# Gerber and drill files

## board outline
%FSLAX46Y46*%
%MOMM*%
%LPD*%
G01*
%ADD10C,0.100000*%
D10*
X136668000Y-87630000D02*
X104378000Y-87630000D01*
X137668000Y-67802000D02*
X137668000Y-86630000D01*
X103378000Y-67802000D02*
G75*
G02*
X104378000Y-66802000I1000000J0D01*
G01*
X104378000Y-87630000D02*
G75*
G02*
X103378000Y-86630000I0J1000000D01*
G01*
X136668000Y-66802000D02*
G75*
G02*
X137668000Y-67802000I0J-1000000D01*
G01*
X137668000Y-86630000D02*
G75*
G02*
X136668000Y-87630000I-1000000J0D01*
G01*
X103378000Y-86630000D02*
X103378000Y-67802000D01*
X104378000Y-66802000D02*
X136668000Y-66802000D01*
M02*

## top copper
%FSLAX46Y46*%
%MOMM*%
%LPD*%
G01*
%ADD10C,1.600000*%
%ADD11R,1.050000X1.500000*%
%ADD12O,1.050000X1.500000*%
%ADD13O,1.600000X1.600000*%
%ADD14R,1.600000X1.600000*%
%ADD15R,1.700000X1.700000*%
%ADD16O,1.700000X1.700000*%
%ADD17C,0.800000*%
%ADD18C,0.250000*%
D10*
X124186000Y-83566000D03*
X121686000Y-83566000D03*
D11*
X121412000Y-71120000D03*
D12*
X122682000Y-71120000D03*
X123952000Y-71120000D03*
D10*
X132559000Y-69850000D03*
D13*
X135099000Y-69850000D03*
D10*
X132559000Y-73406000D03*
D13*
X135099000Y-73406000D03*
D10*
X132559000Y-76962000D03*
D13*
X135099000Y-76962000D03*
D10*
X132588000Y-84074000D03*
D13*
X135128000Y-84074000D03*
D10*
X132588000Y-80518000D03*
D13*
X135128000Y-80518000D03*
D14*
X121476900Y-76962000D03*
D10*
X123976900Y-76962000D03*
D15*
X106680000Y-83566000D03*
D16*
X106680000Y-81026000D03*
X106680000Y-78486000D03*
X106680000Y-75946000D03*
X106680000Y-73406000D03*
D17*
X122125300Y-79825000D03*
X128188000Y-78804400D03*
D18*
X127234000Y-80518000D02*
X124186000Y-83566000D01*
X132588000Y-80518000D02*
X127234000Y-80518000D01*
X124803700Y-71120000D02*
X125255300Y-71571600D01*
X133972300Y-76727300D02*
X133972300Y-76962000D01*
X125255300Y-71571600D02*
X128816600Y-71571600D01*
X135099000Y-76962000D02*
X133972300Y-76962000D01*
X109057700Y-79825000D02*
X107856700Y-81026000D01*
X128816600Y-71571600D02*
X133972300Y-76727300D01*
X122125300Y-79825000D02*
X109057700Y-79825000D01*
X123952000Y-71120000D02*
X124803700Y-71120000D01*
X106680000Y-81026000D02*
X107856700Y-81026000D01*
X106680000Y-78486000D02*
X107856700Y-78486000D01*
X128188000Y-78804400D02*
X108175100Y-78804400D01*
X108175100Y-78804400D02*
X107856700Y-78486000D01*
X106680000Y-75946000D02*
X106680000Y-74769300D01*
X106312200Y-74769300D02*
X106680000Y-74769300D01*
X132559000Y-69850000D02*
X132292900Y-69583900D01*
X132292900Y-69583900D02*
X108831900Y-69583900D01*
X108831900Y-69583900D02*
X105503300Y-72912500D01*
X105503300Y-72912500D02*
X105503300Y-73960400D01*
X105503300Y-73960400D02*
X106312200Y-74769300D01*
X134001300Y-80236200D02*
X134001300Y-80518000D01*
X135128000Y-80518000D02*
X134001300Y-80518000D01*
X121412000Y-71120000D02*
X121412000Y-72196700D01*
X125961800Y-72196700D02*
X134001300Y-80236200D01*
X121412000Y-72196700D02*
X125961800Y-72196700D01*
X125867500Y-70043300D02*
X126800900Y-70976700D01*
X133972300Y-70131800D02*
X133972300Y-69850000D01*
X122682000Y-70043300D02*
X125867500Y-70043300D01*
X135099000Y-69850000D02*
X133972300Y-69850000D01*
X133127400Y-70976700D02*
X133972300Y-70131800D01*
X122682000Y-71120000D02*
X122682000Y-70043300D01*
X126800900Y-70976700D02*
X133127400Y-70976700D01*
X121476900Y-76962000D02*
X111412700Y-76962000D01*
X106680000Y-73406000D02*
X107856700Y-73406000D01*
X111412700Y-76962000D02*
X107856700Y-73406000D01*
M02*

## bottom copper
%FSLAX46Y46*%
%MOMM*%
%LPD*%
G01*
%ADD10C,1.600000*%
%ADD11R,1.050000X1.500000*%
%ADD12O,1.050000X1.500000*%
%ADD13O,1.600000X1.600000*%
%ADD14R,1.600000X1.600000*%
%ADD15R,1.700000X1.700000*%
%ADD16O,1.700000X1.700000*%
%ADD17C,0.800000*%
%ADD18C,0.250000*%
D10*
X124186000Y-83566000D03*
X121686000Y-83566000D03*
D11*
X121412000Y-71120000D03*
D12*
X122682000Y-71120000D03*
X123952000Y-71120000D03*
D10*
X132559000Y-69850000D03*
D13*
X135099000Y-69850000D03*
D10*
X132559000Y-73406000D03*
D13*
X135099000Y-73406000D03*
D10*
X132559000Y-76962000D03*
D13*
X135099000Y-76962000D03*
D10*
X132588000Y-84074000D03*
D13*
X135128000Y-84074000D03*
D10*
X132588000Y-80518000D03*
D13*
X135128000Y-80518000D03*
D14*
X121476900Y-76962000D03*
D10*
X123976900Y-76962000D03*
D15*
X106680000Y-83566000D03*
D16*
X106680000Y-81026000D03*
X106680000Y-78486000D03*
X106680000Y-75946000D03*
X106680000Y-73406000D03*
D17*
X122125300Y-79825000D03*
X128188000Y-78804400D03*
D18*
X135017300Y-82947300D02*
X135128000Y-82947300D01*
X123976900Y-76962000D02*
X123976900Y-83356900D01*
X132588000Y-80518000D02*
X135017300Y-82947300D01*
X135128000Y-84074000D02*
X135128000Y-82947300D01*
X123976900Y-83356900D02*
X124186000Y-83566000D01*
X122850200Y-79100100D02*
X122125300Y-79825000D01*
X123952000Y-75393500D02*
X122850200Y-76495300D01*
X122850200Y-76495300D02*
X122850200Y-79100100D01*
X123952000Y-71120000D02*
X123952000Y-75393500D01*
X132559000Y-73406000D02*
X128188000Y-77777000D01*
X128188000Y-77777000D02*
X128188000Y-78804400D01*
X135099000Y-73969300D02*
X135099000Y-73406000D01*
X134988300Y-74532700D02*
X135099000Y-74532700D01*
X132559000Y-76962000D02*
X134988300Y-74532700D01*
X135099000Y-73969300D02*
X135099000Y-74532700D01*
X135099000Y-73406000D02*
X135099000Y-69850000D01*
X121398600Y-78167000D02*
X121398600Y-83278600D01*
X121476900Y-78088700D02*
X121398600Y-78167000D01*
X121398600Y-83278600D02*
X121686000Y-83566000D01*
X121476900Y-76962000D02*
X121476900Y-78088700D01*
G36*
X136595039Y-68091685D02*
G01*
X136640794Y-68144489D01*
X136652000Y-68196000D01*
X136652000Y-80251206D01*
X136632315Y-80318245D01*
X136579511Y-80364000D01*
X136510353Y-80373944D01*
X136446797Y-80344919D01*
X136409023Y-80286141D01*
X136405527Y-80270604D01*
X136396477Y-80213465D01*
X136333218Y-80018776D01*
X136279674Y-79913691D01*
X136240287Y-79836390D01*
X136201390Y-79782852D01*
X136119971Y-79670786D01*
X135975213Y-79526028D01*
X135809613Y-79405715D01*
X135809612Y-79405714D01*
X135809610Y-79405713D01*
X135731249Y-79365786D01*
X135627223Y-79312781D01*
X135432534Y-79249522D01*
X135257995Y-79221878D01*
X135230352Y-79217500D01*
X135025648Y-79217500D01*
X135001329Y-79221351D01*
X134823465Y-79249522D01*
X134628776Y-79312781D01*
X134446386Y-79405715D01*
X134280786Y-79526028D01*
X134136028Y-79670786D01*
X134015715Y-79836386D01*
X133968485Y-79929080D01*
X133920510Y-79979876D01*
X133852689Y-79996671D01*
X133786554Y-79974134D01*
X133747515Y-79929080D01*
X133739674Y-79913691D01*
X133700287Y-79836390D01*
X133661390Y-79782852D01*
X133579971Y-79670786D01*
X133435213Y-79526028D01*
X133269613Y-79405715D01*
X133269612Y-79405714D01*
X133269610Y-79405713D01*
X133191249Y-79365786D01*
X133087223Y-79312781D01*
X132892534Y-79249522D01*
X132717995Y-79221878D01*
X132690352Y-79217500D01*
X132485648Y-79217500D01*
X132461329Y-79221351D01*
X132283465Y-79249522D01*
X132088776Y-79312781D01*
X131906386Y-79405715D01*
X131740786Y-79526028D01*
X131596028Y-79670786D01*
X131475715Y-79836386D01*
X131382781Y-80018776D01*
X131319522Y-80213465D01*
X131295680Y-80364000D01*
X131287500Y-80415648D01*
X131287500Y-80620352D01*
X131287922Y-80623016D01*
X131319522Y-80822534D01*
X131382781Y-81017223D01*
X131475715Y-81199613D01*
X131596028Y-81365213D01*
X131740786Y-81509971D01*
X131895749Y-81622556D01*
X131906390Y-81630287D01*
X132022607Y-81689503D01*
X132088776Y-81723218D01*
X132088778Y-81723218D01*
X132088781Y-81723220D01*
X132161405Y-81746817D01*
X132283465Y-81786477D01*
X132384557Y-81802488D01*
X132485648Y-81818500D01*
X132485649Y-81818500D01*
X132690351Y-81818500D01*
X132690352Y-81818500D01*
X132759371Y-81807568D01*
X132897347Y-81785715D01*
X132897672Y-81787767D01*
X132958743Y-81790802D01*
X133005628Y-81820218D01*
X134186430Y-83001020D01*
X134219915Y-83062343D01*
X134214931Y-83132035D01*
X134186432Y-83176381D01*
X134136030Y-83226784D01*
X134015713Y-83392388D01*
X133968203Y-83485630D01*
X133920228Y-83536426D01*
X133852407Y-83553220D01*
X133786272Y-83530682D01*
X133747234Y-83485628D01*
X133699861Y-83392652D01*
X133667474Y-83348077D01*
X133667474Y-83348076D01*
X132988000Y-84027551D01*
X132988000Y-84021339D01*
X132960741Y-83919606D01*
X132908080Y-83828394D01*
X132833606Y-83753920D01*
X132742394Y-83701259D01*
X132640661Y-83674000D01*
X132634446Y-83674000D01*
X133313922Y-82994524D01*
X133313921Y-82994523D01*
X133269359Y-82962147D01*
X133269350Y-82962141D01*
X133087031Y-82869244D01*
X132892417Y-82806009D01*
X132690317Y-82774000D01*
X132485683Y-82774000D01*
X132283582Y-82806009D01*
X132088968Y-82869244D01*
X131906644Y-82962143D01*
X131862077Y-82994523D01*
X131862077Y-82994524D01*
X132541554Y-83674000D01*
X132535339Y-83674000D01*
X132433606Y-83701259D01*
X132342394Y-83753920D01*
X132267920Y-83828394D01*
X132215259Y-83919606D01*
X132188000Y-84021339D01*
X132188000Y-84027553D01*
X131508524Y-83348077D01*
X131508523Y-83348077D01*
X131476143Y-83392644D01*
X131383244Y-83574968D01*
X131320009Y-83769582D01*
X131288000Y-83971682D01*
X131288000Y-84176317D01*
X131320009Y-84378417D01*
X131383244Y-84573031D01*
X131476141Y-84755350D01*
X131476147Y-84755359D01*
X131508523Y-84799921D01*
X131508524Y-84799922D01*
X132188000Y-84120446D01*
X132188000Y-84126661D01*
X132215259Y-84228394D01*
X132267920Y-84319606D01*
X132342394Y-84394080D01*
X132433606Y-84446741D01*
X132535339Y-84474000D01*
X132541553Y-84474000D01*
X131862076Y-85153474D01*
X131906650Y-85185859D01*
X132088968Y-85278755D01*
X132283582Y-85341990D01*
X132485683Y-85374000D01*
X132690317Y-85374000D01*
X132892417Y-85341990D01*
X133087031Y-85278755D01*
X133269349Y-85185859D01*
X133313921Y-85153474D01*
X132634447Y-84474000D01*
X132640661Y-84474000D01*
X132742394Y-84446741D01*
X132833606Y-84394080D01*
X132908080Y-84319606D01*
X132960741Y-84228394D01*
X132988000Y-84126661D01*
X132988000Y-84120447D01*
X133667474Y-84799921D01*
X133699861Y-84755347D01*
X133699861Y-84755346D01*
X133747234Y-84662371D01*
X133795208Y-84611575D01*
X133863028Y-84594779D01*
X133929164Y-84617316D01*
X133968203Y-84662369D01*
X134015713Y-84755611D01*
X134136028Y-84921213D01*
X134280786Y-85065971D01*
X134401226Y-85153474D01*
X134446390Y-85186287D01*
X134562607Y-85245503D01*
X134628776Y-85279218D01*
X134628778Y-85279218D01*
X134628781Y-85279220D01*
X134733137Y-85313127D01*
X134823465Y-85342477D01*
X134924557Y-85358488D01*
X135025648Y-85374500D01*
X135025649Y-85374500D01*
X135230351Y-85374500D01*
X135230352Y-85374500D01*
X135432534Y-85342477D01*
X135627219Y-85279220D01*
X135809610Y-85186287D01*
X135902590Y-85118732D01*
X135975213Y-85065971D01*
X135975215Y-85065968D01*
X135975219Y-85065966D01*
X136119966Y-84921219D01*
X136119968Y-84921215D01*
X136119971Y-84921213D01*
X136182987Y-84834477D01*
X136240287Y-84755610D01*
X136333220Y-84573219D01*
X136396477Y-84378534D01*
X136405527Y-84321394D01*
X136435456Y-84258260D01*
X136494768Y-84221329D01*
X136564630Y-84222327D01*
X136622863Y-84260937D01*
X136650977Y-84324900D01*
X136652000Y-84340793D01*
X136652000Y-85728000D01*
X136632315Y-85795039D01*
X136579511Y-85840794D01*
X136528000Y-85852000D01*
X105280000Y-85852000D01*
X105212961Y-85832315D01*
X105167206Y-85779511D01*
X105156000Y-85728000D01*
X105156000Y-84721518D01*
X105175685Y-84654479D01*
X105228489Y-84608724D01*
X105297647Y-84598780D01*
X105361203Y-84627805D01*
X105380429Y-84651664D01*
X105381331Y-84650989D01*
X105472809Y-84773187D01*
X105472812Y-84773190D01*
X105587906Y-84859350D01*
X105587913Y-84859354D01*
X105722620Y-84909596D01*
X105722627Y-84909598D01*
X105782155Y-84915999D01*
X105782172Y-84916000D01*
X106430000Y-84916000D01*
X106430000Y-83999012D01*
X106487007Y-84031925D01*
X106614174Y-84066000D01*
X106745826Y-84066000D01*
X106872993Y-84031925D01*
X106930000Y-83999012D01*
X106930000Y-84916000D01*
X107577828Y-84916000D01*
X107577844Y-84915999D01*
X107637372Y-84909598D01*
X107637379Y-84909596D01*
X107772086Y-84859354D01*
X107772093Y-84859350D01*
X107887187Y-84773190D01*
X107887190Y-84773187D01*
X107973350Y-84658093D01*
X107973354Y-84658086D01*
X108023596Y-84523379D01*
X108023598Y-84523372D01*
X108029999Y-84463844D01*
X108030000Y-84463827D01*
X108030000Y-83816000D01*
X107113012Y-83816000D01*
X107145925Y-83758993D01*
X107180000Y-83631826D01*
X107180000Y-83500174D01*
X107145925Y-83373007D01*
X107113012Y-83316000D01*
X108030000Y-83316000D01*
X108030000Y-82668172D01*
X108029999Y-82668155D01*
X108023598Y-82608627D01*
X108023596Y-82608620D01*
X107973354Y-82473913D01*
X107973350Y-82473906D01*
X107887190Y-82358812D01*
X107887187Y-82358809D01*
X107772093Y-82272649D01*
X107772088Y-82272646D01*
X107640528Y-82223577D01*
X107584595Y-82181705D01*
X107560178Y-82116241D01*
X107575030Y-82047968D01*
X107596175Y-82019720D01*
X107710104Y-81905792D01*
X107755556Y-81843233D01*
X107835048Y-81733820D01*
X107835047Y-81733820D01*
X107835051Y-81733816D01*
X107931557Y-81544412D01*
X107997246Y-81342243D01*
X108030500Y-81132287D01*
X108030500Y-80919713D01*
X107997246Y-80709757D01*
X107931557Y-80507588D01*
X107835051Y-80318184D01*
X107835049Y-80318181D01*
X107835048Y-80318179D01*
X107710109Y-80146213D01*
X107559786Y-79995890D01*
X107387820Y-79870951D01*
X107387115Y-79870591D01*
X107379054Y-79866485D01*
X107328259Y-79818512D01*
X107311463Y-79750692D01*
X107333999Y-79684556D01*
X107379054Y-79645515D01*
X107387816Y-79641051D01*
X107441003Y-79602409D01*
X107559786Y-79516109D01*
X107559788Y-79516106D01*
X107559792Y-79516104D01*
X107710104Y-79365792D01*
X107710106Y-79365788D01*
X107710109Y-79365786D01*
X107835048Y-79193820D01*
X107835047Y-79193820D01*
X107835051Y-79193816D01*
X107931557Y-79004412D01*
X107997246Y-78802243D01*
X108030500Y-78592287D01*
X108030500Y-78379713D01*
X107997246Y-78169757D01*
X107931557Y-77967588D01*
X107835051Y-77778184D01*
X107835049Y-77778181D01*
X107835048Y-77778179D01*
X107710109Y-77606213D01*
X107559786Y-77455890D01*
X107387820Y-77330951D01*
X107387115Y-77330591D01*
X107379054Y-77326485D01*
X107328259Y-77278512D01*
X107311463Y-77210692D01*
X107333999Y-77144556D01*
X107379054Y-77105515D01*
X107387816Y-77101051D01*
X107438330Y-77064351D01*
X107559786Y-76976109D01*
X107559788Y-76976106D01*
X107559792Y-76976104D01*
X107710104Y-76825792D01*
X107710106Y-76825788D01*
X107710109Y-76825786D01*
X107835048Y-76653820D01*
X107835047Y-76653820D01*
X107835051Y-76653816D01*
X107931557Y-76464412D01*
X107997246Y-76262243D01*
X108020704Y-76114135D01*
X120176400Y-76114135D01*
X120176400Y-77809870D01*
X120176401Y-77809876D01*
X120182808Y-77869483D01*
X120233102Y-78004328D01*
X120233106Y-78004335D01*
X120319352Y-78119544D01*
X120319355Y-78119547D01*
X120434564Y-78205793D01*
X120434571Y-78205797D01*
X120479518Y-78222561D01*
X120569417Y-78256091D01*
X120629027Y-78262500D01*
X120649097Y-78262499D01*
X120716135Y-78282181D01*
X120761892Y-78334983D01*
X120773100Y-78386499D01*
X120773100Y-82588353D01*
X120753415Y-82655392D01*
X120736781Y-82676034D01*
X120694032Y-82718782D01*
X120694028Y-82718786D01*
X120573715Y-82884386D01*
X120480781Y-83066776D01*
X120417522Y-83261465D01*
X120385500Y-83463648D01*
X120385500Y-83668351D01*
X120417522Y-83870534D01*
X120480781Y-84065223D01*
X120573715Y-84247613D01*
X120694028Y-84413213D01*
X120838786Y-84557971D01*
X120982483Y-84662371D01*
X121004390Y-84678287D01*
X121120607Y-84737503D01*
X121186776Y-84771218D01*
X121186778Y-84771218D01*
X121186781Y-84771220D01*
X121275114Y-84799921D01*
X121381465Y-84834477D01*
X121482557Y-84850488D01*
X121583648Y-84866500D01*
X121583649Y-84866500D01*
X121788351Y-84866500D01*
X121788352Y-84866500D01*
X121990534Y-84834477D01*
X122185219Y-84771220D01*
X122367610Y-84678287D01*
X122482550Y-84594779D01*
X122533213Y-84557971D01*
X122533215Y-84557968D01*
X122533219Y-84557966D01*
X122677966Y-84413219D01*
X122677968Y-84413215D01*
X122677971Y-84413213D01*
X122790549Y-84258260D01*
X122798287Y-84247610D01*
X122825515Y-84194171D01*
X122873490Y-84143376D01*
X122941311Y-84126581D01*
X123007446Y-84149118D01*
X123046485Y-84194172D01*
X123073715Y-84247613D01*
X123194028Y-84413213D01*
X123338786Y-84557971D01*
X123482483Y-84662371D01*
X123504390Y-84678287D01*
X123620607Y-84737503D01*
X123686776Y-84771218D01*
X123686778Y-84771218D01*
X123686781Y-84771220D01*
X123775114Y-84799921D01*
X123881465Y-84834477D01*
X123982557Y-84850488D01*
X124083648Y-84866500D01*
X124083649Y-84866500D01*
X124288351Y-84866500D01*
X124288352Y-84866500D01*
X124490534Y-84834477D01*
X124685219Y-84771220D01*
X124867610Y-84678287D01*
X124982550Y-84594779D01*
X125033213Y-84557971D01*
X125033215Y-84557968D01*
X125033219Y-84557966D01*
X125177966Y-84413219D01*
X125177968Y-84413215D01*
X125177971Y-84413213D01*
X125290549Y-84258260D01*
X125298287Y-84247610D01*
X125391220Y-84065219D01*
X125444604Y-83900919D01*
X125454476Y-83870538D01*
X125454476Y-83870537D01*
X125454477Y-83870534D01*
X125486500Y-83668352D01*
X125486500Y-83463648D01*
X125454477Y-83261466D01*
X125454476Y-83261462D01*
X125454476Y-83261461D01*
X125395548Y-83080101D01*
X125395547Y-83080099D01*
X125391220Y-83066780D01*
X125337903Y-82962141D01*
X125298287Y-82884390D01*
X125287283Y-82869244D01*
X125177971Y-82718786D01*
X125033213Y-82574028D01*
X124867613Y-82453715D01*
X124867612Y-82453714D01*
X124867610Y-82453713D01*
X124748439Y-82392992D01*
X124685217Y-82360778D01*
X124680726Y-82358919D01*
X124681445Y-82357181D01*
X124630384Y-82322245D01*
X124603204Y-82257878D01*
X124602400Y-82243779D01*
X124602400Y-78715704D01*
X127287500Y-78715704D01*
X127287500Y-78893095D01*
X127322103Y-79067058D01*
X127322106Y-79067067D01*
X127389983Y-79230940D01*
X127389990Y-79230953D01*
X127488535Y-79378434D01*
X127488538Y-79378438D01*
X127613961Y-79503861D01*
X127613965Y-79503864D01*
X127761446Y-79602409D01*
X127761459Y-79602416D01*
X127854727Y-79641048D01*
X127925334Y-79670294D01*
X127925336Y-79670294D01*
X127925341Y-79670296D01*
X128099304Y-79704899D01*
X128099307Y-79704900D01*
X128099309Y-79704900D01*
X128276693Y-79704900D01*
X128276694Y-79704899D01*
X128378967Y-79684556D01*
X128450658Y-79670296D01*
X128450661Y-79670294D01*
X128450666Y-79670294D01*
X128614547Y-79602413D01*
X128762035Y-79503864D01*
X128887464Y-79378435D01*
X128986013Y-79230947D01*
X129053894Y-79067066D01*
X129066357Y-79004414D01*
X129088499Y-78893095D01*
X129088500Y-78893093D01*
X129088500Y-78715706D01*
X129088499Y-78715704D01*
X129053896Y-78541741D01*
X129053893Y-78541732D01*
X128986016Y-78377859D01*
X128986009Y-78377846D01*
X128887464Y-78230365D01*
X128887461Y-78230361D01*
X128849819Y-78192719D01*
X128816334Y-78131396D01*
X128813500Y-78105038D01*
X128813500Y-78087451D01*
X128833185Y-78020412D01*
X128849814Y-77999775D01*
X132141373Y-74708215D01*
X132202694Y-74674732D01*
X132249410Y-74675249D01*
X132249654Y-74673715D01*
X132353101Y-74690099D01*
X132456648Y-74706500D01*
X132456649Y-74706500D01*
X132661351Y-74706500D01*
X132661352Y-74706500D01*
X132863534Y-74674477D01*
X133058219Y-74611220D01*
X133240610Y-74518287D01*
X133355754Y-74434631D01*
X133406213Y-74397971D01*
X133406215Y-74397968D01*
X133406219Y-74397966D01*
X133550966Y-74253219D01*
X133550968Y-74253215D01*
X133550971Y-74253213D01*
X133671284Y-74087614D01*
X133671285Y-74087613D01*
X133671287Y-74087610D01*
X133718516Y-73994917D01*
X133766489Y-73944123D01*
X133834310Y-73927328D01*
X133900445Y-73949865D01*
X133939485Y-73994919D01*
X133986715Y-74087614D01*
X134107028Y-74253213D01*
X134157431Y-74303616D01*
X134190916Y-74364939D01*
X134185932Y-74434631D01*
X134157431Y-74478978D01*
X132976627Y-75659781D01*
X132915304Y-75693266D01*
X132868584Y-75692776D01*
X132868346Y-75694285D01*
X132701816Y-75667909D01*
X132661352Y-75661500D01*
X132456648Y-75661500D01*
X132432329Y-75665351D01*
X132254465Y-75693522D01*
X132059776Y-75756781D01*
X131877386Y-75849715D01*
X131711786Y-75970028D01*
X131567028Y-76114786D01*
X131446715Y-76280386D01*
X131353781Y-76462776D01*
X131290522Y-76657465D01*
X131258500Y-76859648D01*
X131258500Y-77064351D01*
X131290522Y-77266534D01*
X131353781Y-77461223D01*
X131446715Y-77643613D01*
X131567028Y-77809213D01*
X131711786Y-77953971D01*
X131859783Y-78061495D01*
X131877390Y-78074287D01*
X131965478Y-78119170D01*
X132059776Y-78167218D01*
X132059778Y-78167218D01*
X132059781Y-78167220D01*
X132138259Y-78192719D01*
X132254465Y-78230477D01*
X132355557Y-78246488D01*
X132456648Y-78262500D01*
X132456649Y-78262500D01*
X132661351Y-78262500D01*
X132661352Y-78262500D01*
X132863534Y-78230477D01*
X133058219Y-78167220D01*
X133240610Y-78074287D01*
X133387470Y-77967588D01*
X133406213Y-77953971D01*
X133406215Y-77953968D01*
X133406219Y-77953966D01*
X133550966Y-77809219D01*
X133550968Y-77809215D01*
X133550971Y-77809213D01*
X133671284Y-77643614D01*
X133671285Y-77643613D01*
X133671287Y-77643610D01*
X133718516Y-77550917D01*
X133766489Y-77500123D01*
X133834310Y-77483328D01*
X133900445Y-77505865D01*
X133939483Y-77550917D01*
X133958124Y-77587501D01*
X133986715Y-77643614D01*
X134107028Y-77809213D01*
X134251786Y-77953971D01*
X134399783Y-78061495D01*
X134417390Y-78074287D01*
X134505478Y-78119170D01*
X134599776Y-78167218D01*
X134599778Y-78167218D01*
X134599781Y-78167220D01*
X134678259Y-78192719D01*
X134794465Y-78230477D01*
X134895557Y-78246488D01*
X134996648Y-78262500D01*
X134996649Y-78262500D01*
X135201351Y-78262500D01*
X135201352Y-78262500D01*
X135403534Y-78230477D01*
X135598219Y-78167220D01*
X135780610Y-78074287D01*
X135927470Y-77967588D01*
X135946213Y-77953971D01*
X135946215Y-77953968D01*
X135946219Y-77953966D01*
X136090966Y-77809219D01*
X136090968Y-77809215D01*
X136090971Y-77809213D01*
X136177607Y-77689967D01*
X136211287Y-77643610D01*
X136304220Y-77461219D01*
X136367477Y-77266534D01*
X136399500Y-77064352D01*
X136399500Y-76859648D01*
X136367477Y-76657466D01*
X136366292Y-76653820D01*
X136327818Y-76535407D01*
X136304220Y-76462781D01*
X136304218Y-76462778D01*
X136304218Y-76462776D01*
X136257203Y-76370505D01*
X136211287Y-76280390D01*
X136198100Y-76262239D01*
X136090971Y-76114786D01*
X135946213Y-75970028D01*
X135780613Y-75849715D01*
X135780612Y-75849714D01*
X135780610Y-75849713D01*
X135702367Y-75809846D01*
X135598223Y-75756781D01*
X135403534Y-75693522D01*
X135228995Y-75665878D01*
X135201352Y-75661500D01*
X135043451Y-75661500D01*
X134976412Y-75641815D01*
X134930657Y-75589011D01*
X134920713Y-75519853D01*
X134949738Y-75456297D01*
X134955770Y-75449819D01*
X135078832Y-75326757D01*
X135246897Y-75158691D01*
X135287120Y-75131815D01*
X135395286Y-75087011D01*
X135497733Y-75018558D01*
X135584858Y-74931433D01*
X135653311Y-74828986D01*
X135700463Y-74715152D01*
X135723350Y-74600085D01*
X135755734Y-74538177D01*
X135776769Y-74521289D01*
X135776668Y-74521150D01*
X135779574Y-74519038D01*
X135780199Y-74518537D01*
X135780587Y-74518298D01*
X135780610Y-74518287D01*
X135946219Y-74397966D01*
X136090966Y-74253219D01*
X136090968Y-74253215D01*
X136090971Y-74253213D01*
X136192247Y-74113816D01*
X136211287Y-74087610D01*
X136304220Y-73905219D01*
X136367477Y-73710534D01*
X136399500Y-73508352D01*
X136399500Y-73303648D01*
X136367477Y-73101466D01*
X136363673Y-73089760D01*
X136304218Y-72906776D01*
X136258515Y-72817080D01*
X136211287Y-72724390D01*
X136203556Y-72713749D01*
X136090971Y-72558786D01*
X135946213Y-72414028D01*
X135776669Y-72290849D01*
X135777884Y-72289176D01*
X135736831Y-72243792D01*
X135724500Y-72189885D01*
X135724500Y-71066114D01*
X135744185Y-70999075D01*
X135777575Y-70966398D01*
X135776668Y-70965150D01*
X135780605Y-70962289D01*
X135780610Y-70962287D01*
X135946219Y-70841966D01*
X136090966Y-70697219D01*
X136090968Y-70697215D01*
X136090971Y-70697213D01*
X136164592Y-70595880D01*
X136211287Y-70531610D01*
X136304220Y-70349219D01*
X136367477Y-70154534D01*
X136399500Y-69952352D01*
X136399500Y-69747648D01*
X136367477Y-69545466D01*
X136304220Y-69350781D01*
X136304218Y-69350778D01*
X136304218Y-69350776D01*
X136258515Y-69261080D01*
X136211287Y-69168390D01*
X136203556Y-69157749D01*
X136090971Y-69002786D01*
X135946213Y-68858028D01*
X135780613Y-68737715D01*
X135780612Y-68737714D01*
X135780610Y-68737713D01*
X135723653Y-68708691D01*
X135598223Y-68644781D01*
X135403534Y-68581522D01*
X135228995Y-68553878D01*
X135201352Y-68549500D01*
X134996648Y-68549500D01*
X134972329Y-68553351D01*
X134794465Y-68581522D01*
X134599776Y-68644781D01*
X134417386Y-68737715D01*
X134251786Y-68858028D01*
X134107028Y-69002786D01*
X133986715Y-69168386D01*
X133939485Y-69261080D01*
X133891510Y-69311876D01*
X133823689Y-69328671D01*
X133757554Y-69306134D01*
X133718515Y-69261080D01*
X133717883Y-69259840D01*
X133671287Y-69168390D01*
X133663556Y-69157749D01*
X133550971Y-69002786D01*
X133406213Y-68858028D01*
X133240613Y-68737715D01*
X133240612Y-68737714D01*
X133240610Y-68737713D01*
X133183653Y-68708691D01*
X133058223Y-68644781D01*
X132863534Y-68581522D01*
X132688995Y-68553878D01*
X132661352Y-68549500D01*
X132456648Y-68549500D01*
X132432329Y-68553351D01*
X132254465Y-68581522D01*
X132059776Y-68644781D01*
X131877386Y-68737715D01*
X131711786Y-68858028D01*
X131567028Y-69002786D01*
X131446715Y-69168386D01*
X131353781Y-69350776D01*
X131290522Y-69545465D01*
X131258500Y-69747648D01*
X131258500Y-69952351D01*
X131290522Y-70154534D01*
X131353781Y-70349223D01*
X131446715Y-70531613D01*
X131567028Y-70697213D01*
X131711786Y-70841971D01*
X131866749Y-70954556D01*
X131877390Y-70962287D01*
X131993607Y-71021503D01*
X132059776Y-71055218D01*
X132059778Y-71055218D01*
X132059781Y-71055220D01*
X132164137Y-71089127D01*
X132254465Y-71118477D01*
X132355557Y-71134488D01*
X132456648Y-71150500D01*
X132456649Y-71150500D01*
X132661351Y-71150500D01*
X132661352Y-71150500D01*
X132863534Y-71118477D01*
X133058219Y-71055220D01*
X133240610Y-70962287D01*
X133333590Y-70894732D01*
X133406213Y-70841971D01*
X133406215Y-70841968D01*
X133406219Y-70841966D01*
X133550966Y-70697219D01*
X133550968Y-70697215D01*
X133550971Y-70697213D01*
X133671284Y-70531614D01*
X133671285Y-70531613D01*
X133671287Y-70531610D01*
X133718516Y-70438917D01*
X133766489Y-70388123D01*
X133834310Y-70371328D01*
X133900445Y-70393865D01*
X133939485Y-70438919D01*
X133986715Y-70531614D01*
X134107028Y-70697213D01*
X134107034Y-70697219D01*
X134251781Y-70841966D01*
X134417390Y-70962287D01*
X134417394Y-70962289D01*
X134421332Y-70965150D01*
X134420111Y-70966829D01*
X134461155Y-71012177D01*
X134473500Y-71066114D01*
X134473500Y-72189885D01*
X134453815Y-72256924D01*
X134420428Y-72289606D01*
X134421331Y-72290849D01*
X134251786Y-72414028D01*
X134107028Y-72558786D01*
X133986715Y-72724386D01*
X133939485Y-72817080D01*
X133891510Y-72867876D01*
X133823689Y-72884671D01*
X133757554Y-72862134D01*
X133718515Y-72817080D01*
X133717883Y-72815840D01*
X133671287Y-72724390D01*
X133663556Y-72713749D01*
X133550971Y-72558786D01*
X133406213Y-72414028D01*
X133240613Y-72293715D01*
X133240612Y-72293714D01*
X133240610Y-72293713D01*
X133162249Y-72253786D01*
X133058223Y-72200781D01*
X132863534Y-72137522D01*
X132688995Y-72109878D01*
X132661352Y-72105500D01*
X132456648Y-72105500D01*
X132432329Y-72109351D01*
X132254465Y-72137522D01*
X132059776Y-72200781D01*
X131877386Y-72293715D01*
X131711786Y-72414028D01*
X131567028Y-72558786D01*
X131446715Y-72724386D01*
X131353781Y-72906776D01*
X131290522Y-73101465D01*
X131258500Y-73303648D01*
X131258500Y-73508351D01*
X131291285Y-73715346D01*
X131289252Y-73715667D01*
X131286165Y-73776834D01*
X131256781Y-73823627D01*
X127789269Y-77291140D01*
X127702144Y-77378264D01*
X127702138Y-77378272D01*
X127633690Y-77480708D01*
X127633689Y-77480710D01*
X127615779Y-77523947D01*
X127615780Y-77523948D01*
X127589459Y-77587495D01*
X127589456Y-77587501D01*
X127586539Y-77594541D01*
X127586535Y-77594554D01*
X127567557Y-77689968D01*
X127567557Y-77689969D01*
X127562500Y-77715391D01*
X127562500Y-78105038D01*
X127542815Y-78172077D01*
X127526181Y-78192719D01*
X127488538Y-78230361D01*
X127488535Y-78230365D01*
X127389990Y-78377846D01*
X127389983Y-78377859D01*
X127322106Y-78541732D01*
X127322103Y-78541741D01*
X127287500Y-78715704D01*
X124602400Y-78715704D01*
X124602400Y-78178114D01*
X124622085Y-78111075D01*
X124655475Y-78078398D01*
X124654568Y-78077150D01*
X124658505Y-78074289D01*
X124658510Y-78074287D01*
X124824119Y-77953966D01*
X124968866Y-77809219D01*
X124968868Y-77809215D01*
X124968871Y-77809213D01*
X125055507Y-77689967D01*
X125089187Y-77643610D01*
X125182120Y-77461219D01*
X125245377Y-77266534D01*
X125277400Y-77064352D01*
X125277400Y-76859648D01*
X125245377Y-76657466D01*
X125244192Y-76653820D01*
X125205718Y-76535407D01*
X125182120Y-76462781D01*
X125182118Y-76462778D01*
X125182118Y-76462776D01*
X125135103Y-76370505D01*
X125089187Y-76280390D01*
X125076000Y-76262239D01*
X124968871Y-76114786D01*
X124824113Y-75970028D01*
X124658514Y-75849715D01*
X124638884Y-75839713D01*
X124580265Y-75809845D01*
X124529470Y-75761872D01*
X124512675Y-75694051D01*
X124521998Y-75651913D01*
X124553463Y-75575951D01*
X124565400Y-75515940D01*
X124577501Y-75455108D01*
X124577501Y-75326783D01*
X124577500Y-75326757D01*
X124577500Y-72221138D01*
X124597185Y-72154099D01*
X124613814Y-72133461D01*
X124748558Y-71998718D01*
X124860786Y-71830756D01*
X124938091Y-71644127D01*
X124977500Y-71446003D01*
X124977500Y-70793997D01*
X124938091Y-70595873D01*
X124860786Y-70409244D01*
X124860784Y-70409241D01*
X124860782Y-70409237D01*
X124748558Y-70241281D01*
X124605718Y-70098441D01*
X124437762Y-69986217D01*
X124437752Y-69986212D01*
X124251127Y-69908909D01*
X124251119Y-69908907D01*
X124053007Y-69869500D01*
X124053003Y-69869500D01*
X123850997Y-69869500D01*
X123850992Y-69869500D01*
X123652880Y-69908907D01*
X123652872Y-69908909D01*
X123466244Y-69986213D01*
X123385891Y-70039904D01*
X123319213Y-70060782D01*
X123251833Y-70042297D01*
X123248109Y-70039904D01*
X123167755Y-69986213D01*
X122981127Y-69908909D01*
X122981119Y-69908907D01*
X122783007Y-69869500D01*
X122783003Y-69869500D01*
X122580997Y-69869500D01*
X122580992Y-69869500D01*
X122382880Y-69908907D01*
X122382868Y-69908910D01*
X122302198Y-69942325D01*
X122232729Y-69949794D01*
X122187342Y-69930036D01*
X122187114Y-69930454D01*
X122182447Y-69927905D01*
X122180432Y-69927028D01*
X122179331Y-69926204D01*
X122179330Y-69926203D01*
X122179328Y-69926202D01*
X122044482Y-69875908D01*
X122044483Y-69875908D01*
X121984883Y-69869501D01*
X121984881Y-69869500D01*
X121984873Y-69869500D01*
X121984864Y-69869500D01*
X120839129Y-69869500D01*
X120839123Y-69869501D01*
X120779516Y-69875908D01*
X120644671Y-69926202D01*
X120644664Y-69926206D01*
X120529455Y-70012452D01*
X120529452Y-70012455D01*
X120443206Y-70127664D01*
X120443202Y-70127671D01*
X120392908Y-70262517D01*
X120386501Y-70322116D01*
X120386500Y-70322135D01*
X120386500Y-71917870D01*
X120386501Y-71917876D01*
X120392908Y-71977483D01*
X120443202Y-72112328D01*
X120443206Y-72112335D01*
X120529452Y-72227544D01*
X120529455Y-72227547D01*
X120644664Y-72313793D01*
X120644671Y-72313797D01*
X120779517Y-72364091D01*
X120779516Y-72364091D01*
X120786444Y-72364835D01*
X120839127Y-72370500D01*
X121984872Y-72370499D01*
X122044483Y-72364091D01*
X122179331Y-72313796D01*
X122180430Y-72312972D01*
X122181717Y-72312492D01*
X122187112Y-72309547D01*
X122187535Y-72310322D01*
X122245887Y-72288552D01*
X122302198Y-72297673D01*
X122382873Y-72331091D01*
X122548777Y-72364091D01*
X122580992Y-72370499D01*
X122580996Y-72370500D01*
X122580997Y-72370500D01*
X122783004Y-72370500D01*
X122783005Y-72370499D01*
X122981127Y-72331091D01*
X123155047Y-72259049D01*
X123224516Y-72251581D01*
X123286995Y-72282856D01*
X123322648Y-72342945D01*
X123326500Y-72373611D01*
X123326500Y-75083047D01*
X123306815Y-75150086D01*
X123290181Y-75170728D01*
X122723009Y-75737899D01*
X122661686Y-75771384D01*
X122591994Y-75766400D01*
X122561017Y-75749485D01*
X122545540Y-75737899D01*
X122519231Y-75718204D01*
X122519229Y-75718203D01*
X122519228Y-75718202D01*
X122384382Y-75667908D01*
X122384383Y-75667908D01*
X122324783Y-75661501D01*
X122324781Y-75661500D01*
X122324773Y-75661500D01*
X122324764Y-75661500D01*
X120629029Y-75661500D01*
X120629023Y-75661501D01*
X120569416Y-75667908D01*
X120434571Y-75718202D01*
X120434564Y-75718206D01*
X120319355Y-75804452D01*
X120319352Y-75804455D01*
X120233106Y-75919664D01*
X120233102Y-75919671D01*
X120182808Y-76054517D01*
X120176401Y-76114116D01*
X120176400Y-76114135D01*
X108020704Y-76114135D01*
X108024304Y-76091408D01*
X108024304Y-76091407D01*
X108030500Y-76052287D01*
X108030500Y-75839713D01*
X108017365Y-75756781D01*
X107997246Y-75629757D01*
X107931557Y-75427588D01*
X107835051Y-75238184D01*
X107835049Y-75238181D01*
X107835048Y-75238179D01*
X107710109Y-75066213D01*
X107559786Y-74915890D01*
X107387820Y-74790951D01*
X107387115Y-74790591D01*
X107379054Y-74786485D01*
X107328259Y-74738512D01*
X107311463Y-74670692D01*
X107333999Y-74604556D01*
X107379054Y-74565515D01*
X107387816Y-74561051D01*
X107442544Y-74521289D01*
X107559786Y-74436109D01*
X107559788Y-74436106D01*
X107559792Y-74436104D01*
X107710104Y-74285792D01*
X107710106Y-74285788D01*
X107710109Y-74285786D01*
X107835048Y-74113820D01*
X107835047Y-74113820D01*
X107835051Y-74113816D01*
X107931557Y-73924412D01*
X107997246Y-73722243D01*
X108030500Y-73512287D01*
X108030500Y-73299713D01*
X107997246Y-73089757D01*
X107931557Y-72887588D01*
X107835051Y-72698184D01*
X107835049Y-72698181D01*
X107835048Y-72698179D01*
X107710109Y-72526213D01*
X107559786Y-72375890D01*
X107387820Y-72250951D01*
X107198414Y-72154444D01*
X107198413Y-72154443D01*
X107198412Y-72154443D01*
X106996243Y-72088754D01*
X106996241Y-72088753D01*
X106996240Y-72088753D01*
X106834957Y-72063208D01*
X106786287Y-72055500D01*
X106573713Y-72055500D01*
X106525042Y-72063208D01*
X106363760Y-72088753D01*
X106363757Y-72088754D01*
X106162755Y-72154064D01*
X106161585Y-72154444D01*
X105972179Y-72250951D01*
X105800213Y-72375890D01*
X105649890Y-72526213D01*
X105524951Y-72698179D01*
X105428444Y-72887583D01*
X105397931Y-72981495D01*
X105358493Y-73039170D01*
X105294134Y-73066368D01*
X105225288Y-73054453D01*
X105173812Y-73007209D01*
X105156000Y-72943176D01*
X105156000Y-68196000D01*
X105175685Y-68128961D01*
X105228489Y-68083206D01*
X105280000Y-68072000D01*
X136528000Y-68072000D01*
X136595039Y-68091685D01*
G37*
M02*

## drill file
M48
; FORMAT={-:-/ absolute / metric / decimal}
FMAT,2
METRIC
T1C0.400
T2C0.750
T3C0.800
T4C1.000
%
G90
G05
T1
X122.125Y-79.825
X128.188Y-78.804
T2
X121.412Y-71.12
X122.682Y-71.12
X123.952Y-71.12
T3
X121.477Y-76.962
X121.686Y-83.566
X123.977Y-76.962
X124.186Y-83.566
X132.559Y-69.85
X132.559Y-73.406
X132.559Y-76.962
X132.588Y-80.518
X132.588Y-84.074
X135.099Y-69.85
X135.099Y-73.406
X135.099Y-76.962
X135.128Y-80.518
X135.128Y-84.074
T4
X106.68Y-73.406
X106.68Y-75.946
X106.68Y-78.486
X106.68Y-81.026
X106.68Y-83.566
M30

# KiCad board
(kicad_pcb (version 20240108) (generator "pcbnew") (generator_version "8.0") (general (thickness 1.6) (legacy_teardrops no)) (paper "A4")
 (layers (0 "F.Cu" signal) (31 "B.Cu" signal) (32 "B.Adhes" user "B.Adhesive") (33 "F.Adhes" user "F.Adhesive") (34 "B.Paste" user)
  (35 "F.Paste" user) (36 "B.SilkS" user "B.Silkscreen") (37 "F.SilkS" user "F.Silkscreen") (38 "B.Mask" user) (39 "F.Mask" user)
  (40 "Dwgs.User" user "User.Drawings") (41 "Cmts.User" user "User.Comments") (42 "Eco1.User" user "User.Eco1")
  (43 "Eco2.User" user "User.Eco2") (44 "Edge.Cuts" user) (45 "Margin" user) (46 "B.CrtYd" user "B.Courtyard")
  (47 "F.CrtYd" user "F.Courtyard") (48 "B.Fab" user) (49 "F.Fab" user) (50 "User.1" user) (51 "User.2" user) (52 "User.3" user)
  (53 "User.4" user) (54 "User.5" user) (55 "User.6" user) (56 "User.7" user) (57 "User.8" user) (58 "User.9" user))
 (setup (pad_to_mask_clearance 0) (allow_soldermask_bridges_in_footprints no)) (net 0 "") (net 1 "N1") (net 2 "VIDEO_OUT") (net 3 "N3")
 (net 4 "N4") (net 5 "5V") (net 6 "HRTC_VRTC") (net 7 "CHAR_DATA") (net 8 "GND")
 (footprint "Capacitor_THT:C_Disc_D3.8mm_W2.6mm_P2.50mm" (layer "F.Cu") (at 124.186 83.566 180)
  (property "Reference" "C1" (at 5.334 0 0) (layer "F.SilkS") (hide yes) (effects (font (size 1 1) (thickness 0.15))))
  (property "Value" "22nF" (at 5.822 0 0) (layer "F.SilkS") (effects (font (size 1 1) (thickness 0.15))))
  (pad "1" thru_hole circle (at 0 0 180) (size 1.6 1.6) (drill 0.8) (layers "*.Cu" "*.Mask") (remove_unused_layers no) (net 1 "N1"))
  (pad "2" thru_hole circle (at 2.5 0 180) (size 1.6 1.6) (drill 0.8) (layers "*.Cu" "*.Mask") (remove_unused_layers no) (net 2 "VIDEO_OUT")))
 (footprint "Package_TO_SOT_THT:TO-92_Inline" (layer "F.Cu") (at 121.412 71.12)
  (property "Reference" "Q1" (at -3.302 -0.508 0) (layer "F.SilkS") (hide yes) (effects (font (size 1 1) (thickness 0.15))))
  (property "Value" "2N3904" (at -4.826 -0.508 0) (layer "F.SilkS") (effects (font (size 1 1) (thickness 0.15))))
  (pad "1" thru_hole rect (at 0 0) (size 1.05 1.5) (drill 0.75) (layers "*.Cu" "*.Mask") (remove_unused_layers no) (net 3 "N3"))
  (pad "2" thru_hole oval (at 1.27 0) (size 1.05 1.5) (drill 0.75) (layers "*.Cu" "*.Mask") (remove_unused_layers no) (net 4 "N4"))
  (pad "3" thru_hole oval (at 2.54 0) (size 1.05 1.5) (drill 0.75) (layers "*.Cu" "*.Mask") (remove_unused_layers no) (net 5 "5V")))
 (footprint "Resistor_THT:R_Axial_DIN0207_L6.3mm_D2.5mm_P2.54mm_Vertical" (layer "F.Cu") (at 132.559 69.85)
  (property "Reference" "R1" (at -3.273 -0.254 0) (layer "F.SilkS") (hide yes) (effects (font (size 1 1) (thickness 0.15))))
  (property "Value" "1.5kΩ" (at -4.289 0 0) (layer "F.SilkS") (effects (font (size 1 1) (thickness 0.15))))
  (pad "1" thru_hole circle (at 0 0) (size 1.6 1.6) (drill 0.8) (layers "*.Cu" "*.Mask") (remove_unused_layers no) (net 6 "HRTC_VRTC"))
  (pad "2" thru_hole oval (at 2.54 0) (size 1.6 1.6) (drill 0.8) (layers "*.Cu" "*.Mask") (remove_unused_layers no) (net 4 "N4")))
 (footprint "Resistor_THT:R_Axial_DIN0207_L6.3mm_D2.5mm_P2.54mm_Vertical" (layer "F.Cu") (at 132.559 73.406)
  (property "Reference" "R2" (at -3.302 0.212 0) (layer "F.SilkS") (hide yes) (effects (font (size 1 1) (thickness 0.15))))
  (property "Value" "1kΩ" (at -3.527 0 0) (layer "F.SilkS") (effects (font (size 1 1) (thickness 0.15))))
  (pad "1" thru_hole circle (at 0 0) (size 1.6 1.6) (drill 0.8) (layers "*.Cu" "*.Mask") (remove_unused_layers no) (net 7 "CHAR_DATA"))
  (pad "2" thru_hole oval (at 2.54 0) (size 1.6 1.6) (drill 0.8) (layers "*.Cu" "*.Mask") (remove_unused_layers no) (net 4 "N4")))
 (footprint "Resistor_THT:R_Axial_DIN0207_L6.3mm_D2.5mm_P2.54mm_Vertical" (layer "F.Cu") (at 132.559 76.962)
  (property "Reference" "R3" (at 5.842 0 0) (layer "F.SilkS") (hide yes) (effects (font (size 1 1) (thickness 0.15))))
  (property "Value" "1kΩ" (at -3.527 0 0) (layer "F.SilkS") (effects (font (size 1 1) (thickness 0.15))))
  (pad "1" thru_hole circle (at 0 0) (size 1.6 1.6) (drill 0.8) (layers "*.Cu" "*.Mask") (remove_unused_layers no) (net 4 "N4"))
  (pad "2" thru_hole oval (at 2.54 0) (size 1.6 1.6) (drill 0.8) (layers "*.Cu" "*.Mask") (remove_unused_layers no) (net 5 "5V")))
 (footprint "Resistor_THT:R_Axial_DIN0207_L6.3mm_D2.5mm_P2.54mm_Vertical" (layer "F.Cu") (at 132.588 84.074)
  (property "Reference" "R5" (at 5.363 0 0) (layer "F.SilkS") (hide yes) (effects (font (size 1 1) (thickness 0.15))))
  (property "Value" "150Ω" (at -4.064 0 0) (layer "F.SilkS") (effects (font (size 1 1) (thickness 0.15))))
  (pad "1" thru_hole circle (at 0 0) (size 1.6 1.6) (drill 0.8) (layers "*.Cu" "*.Mask") (remove_unused_layers no) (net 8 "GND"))
  (pad "2" thru_hole oval (at 2.54 0) (size 1.6 1.6) (drill 0.8) (layers "*.Cu" "*.Mask") (remove_unused_layers no) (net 1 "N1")))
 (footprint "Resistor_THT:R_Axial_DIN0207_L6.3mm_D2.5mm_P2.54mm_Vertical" (layer "F.Cu") (at 132.588 80.518)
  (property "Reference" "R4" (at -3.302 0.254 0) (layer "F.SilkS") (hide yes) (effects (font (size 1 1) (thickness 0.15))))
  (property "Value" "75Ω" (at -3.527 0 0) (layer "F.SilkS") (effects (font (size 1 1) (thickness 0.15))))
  (pad "1" thru_hole circle (at 0 0) (size 1.6 1.6) (drill 0.8) (layers "*.Cu" "*.Mask") (remove_unused_layers no) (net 1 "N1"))
  (pad "2" thru_hole oval (at 2.54 0) (size 1.6 1.6) (drill 0.8) (layers "*.Cu" "*.Mask") (remove_unused_layers no) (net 3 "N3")))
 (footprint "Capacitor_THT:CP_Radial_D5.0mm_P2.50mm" (layer "F.Cu") (at 121.4769 76.962)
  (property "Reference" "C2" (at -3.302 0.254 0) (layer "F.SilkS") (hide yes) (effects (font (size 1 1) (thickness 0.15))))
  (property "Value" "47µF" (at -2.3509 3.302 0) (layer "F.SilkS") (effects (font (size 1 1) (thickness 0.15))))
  (pad "1" thru_hole rect (at 0 0) (size 1.6 1.6) (drill 0.8) (layers "*.Cu" "*.Mask") (remove_unused_layers no) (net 2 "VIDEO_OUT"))
  (pad "2" thru_hole circle (at 2.5 0) (size 1.6 1.6) (drill 0.8) (layers "*.Cu" "*.Mask") (remove_unused_layers no) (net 1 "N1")))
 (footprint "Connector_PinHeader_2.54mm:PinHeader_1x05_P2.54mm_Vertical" (layer "F.Cu") (at 106.68 83.566 180)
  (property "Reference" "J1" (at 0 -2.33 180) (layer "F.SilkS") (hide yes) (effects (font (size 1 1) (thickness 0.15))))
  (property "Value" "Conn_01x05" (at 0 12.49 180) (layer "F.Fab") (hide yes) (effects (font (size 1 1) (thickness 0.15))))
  (pad "1" thru_hole rect (at 0 0 180) (size 1.7 1.7) (drill 1) (layers "*.Cu" "*.Mask") (remove_unused_layers no) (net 8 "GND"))
  (pad "2" thru_hole oval (at 0 2.54 180) (size 1.7 1.7) (drill 1) (layers "*.Cu" "*.Mask") (remove_unused_layers no) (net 5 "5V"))
  (pad "3" thru_hole oval (at 0 5.08 180) (size 1.7 1.7) (drill 1) (layers "*.Cu" "*.Mask") (remove_unused_layers no) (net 7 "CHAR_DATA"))
  (pad "4" thru_hole oval (at 0 7.62 180) (size 1.7 1.7) (drill 1) (layers "*.Cu" "*.Mask") (remove_unused_layers no) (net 6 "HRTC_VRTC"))
  (pad "5" thru_hole oval (at 0 10.16 180) (size 1.7 1.7) (drill 1) (layers "*.Cu" "*.Mask") (remove_unused_layers no) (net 2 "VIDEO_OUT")))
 (gr_line (start 136.668 87.63) (end 104.378 87.63) (stroke (width 0.1) (type default)) (layer "Edge.Cuts"))
 (gr_line (start 137.668 67.802) (end 137.668 86.63) (stroke (width 0.1) (type default)) (layer "Edge.Cuts"))
 (gr_arc (start 103.378 67.802) (mid 103.670893 67.094893) (end 104.378 66.802) (stroke (width 0.1) (type default)) (layer "Edge.Cuts"))
 (gr_arc (start 104.378 87.63) (mid 103.670893 87.337107) (end 103.378 86.63) (stroke (width 0.1) (type default)) (layer "Edge.Cuts"))
 (gr_arc (start 136.668 66.802) (mid 137.375107 67.094893) (end 137.668 67.802) (stroke (width 0.1) (type default)) (layer "Edge.Cuts"))
 (gr_arc (start 137.668 86.63) (mid 137.375107 87.337107) (end 136.668 87.63) (stroke (width 0.1) (type default)) (layer "Edge.Cuts"))
 (gr_line (start 103.378 86.63) (end 103.378 67.802) (stroke (width 0.1) (type default)) (layer "Edge.Cuts"))
 (gr_line (start 104.378 66.802) (end 136.668 66.802) (stroke (width 0.1) (type default)) (layer "Edge.Cuts"))
 (segment (start 127.234 80.518) (end 124.186 83.566) (width 0.25) (layer "F.Cu") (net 1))
 (segment (start 132.588 80.518) (end 127.234 80.518) (width 0.25) (layer "F.Cu") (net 1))
 (segment (start 135.0173 82.9473) (end 135.128 82.9473) (width 0.25) (layer "B.Cu") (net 1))
 (segment (start 123.9769 76.962) (end 123.9769 83.3569) (width 0.25) (layer "B.Cu") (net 1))
 (segment (start 132.588 80.518) (end 135.0173 82.9473) (width 0.25) (layer "B.Cu") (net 1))
 (segment (start 135.128 84.074) (end 135.128 82.9473) (width 0.25) (layer "B.Cu") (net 1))
 (segment (start 123.9769 83.3569) (end 124.186 83.566) (width 0.25) (layer "B.Cu") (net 1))
 (segment (start 124.8037 71.12) (end 125.2553 71.5716) (width 0.25) (layer "F.Cu") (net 5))
 (segment (start 133.9723 76.7273) (end 133.9723 76.962) (width 0.25) (layer "F.Cu") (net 5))
 (segment (start 125.2553 71.5716) (end 128.8166 71.5716) (width 0.25) (layer "F.Cu") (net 5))
 (segment (start 135.099 76.962) (end 133.9723 76.962) (width 0.25) (layer "F.Cu") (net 5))
 (segment (start 109.0577 79.825) (end 107.8567 81.026) (width 0.25) (layer "F.Cu") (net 5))
 (segment (start 128.8166 71.5716) (end 133.9723 76.7273) (width 0.25) (layer "F.Cu") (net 5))
 (segment (start 122.1253 79.825) (end 109.0577 79.825) (width 0.25) (layer "F.Cu") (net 5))
 (segment (start 123.952 71.12) (end 124.8037 71.12) (width 0.25) (layer "F.Cu") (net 5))
 (segment (start 106.68 81.026) (end 107.8567 81.026) (width 0.25) (layer "F.Cu") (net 5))
 (via (at 122.1253 79.825) (size 0.8) (drill 0.4) (layers "F.Cu" "B.Cu") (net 5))
 (segment (start 122.8502 79.1001) (end 122.1253 79.825) (width 0.25) (layer "B.Cu") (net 5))
 (segment (start 123.952 75.3935) (end 122.8502 76.4953) (width 0.25) (layer "B.Cu") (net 5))
 (segment (start 122.8502 76.4953) (end 122.8502 79.1001) (width 0.25) (layer "B.Cu") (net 5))
 (segment (start 123.952 71.12) (end 123.952 75.3935) (width 0.25) (layer "B.Cu") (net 5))
 (segment (start 106.68 78.486) (end 107.8567 78.486) (width 0.25) (layer "F.Cu") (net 7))
 (segment (start 128.188 78.8044) (end 108.1751 78.8044) (width 0.25) (layer "F.Cu") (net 7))
 (segment (start 108.1751 78.8044) (end 107.8567 78.486) (width 0.25) (layer "F.Cu") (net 7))
 (via (at 128.188 78.8044) (size 0.8) (drill 0.4) (layers "F.Cu" "B.Cu") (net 7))
 (segment (start 132.559 73.406) (end 128.188 77.777) (width 0.25) (layer "B.Cu") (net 7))
 (segment (start 128.188 77.777) (end 128.188 78.8044) (width 0.25) (layer "B.Cu") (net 7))
 (segment (start 106.68 75.946) (end 106.68 74.7693) (width 0.25) (layer "F.Cu") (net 6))
 (segment (start 106.3122 74.7693) (end 106.68 74.7693) (width 0.25) (layer "F.Cu") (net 6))
 (segment (start 132.559 69.85) (end 132.2929 69.5839) (width 0.25) (layer "F.Cu") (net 6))
 (segment (start 132.2929 69.5839) (end 108.8319 69.5839) (width 0.25) (layer "F.Cu") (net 6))
 (segment (start 108.8319 69.5839) (end 105.5033 72.9125) (width 0.25) (layer "F.Cu") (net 6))
 (segment (start 105.5033 72.9125) (end 105.5033 73.9604) (width 0.25) (layer "F.Cu") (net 6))
 (segment (start 105.5033 73.9604) (end 106.3122 74.7693) (width 0.25) (layer "F.Cu") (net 6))
 (segment (start 134.0013 80.2362) (end 134.0013 80.518) (width 0.25) (layer "F.Cu") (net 3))
 (segment (start 135.128 80.518) (end 134.0013 80.518) (width 0.25) (layer "F.Cu") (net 3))
 (segment (start 121.412 71.12) (end 121.412 72.1967) (width 0.25) (layer "F.Cu") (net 3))
 (segment (start 125.9618 72.1967) (end 134.0013 80.2362) (width 0.25) (layer "F.Cu") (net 3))
 (segment (start 121.412 72.1967) (end 125.9618 72.1967) (width 0.25) (layer "F.Cu") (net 3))
 (segment (start 125.8675 70.0433) (end 126.8009 70.9767) (width 0.25) (layer "F.Cu") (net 4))
 (segment (start 133.9723 70.1318) (end 133.9723 69.85) (width 0.25) (layer "F.Cu") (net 4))
 (segment (start 122.682 70.0433) (end 125.8675 70.0433) (width 0.25) (layer "F.Cu") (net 4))
 (segment (start 135.099 69.85) (end 133.9723 69.85) (width 0.25) (layer "F.Cu") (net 4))
 (segment (start 133.1274 70.9767) (end 133.9723 70.1318) (width 0.25) (layer "F.Cu") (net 4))
 (segment (start 122.682 71.12) (end 122.682 70.0433) (width 0.25) (layer "F.Cu") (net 4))
 (segment (start 126.8009 70.9767) (end 133.1274 70.9767) (width 0.25) (layer "F.Cu") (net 4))
 (segment (start 135.099 73.9693) (end 135.099 73.406) (width 0.25) (layer "B.Cu") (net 4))
 (segment (start 134.9883 74.5327) (end 135.099 74.5327) (width 0.25) (layer "B.Cu") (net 4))
 (segment (start 132.559 76.962) (end 134.9883 74.5327) (width 0.25) (layer "B.Cu") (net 4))
 (segment (start 135.099 73.9693) (end 135.099 74.5327) (width 0.25) (layer "B.Cu") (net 4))
 (segment (start 135.099 73.406) (end 135.099 69.85) (width 0.25) (layer "B.Cu") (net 4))
 (segment (start 121.4769 76.962) (end 111.4127 76.962) (width 0.25) (layer "F.Cu") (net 2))
 (segment (start 106.68 73.406) (end 107.8567 73.406) (width 0.25) (layer "F.Cu") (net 2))
 (segment (start 111.4127 76.962) (end 107.8567 73.406) (width 0.25) (layer "F.Cu") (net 2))
 (segment (start 121.3986 78.167) (end 121.3986 83.2786) (width 0.25) (layer "B.Cu") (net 2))
 (segment (start 121.4769 78.0887) (end 121.3986 78.167) (width 0.25) (layer "B.Cu") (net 2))
 (segment (start 121.3986 83.2786) (end 121.686 83.566) (width 0.25) (layer "B.Cu") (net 2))
 (segment (start 121.4769 76.962) (end 121.4769 78.0887) (width 0.25) (layer "B.Cu") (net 2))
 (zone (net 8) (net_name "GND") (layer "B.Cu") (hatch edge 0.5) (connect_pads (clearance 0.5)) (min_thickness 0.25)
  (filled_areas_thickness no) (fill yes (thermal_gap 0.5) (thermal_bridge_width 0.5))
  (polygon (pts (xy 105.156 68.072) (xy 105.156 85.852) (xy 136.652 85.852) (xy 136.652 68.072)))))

